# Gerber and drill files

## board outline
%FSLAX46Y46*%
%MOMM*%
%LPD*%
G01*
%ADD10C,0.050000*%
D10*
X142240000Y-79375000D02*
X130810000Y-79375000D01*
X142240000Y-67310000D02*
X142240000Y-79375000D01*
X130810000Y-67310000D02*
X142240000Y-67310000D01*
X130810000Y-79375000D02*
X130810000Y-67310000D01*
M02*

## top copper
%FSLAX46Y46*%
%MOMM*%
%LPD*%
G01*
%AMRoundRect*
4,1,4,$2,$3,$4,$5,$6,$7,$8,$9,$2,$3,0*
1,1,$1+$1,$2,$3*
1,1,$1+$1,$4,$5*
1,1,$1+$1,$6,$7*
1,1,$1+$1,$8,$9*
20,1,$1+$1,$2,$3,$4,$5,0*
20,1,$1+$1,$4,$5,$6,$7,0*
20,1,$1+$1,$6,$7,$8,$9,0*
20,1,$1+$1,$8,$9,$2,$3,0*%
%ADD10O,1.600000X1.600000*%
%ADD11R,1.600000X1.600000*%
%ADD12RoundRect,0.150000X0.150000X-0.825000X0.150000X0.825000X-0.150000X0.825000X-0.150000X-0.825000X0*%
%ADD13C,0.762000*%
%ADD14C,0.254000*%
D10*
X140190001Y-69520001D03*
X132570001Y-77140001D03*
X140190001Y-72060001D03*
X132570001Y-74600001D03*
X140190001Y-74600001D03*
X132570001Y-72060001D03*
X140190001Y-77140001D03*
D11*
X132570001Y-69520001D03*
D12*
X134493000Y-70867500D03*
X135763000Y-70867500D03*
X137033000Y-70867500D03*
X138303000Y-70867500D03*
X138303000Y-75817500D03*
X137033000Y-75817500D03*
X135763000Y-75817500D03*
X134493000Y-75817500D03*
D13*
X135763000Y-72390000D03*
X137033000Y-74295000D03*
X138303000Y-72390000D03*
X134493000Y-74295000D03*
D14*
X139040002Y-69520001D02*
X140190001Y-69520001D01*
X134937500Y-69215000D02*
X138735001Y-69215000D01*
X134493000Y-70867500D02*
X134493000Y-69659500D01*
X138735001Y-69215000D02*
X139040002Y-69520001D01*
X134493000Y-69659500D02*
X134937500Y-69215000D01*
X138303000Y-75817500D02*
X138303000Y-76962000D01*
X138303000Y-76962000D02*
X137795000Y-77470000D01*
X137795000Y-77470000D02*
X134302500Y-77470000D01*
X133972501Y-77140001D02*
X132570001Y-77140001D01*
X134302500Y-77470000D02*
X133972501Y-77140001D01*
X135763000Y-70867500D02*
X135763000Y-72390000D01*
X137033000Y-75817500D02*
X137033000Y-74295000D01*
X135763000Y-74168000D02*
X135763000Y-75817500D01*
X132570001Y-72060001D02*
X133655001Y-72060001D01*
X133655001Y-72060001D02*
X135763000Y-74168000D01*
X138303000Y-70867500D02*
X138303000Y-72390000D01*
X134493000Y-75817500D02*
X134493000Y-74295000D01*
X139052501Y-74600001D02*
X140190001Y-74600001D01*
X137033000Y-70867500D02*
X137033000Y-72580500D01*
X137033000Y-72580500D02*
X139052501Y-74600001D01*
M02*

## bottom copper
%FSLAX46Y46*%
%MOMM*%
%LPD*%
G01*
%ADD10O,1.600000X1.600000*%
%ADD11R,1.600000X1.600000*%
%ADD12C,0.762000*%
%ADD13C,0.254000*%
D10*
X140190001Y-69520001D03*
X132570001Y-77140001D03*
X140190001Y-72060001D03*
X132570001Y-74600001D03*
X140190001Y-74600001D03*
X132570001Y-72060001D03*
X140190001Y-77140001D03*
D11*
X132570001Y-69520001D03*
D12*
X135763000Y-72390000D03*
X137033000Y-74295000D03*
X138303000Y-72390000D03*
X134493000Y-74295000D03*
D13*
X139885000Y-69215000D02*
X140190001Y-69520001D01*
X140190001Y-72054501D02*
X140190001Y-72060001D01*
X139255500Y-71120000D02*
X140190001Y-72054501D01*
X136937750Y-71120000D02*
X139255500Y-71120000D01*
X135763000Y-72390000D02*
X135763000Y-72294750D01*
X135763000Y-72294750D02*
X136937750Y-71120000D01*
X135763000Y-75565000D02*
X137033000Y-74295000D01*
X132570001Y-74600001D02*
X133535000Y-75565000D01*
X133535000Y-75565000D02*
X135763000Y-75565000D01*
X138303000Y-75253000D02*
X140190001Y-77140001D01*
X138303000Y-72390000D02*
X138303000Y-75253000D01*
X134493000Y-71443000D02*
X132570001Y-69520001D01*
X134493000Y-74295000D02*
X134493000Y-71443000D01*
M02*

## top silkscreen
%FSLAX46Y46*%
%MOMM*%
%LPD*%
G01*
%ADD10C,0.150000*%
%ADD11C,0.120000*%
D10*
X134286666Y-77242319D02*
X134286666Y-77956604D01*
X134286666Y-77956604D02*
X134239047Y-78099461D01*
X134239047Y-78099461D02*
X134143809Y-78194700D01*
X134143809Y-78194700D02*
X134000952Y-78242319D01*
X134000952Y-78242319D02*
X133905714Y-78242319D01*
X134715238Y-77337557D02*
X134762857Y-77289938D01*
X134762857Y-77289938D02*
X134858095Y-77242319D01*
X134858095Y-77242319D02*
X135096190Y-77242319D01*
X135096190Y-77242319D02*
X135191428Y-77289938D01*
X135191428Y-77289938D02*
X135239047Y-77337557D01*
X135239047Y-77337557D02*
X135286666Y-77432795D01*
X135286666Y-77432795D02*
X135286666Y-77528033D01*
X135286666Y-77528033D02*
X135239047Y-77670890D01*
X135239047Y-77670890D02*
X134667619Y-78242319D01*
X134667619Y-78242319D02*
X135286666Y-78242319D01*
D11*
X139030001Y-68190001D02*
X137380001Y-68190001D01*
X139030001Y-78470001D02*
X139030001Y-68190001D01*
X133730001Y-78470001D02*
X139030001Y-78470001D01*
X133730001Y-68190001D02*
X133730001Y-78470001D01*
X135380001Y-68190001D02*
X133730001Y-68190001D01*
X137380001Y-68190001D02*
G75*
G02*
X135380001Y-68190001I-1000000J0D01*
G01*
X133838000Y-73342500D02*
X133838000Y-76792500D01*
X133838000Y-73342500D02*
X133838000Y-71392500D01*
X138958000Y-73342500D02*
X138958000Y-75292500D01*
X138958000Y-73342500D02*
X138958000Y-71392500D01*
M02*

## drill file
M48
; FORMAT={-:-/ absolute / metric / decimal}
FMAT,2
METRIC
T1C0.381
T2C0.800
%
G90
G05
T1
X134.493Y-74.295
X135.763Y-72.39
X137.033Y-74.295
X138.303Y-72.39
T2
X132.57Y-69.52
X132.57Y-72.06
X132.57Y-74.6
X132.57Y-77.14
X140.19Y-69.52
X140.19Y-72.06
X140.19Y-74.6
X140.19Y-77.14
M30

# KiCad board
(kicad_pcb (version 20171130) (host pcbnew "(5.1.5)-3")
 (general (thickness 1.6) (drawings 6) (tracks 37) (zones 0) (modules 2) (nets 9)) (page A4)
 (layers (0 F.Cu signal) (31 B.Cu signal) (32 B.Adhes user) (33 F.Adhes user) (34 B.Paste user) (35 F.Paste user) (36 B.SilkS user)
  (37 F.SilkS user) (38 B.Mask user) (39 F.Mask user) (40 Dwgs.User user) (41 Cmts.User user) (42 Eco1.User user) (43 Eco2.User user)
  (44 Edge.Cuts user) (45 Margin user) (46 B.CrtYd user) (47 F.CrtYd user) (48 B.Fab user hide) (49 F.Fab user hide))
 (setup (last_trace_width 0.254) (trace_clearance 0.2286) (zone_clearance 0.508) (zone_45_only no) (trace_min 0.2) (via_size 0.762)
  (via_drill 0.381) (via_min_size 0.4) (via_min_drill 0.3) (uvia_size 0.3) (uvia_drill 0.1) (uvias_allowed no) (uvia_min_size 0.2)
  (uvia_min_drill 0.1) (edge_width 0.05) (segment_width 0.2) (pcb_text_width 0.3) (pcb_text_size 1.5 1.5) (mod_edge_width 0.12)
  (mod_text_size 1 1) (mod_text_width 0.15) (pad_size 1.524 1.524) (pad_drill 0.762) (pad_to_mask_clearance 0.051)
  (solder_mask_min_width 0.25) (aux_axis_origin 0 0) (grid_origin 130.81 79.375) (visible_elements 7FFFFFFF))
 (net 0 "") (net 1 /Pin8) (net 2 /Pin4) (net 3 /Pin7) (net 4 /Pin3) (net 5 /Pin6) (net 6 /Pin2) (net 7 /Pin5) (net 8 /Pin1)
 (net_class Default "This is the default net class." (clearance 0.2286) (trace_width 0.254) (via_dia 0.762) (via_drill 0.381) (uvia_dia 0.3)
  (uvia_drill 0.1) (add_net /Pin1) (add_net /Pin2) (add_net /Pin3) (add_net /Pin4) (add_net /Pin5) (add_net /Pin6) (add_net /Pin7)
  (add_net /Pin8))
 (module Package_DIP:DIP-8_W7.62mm (layer F.Cu) (at 132.570001 69.520001)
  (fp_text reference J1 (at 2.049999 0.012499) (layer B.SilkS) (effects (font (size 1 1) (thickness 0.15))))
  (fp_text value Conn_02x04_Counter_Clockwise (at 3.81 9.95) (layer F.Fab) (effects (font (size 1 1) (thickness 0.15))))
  (fp_line (start 6.46 -1.33) (end 4.81 -1.33) (layer F.SilkS) (width 0.12))
  (fp_line (start 6.46 8.95) (end 6.46 -1.33) (layer F.SilkS) (width 0.12))
  (fp_line (start 1.16 8.95) (end 6.46 8.95) (layer F.SilkS) (width 0.12))
  (fp_line (start 1.16 -1.33) (end 1.16 8.95) (layer F.SilkS) (width 0.12))
  (fp_line (start 2.81 -1.33) (end 1.16 -1.33) (layer F.SilkS) (width 0.12))
  (fp_arc (start 3.81 -1.33) (end 2.81 -1.33) (angle -180) (layer F.SilkS) (width 0.12))
  (pad 8 thru_hole oval (at 7.62 0) (size 1.6 1.6) (drill 0.8) (layers *.Cu *.Mask) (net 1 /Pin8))
  (pad 4 thru_hole oval (at 0 7.62) (size 1.6 1.6) (drill 0.8) (layers *.Cu *.Mask) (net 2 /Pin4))
  (pad 7 thru_hole oval (at 7.62 2.54) (size 1.6 1.6) (drill 0.8) (layers *.Cu *.Mask) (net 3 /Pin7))
  (pad 3 thru_hole oval (at 0 5.08) (size 1.6 1.6) (drill 0.8) (layers *.Cu *.Mask) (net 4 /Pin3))
  (pad 6 thru_hole oval (at 7.62 5.08) (size 1.6 1.6) (drill 0.8) (layers *.Cu *.Mask) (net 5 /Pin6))
  (pad 2 thru_hole oval (at 0 2.54) (size 1.6 1.6) (drill 0.8) (layers *.Cu *.Mask) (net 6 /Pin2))
  (pad 5 thru_hole oval (at 7.62 7.62) (size 1.6 1.6) (drill 0.8) (layers *.Cu *.Mask) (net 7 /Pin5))
  (pad 1 thru_hole rect (at 0 0) (size 1.6 1.6) (drill 0.8) (layers *.Cu *.Mask) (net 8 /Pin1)))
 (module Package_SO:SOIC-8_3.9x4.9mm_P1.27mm (layer F.Cu) (at 136.398 73.3425 90)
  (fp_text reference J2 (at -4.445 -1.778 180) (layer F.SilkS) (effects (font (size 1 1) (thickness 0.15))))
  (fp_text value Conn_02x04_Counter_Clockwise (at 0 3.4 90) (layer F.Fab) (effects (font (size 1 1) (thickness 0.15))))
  (fp_line (start 0 -2.56) (end -3.45 -2.56) (layer F.SilkS) (width 0.12))
  (fp_line (start 0 -2.56) (end 1.95 -2.56) (layer F.SilkS) (width 0.12))
  (fp_line (start 0 2.56) (end -1.95 2.56) (layer F.SilkS) (width 0.12))
  (fp_line (start 0 2.56) (end 1.95 2.56) (layer F.SilkS) (width 0.12))
  (pad 8 smd roundrect (at 2.475 -1.905 90) (size 1.95 0.6) (layers F.Cu F.Paste F.Mask) (roundrect_rratio 0.25) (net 1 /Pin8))
  (pad 7 smd roundrect (at 2.475 -0.635 90) (size 1.95 0.6) (layers F.Cu F.Paste F.Mask) (roundrect_rratio 0.25) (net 3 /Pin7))
  (pad 6 smd roundrect (at 2.475 0.635 90) (size 1.95 0.6) (layers F.Cu F.Paste F.Mask) (roundrect_rratio 0.25) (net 5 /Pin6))
  (pad 5 smd roundrect (at 2.475 1.905 90) (size 1.95 0.6) (layers F.Cu F.Paste F.Mask) (roundrect_rratio 0.25) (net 7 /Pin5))
  (pad 4 smd roundrect (at -2.475 1.905 90) (size 1.95 0.6) (layers F.Cu F.Paste F.Mask) (roundrect_rratio 0.25) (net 2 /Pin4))
  (pad 3 smd roundrect (at -2.475 0.635 90) (size 1.95 0.6) (layers F.Cu F.Paste F.Mask) (roundrect_rratio 0.25) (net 4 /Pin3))
  (pad 2 smd roundrect (at -2.475 -0.635 90) (size 1.95 0.6) (layers F.Cu F.Paste F.Mask) (roundrect_rratio 0.25) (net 6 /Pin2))
  (pad 1 smd roundrect (at -2.475 -1.905 90) (size 1.95 0.6) (layers F.Cu F.Paste F.Mask) (roundrect_rratio 0.25) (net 8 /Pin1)))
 (gr_line (start 142.24 79.375) (end 130.81 79.375) (layer Edge.Cuts) (width 0.05))
 (gr_line (start 142.24 67.31) (end 142.24 79.375) (layer Edge.Cuts) (width 0.05))
 (gr_line (start 130.81 67.31) (end 142.24 67.31) (layer Edge.Cuts) (width 0.05))
 (gr_line (start 130.81 79.375) (end 130.81 67.31) (layer Edge.Cuts) (width 0.05))
 (segment (start 139.885 69.215) (end 140.190001 69.520001) (width 0.254) (layer B.Cu) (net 1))
 (segment (start 139.040002 69.520001) (end 140.190001 69.520001) (width 0.254) (layer F.Cu) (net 1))
 (segment (start 134.9375 69.215) (end 138.735001 69.215) (width 0.254) (layer F.Cu) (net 1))
 (segment (start 134.493 70.8675) (end 134.493 69.6595) (width 0.254) (layer F.Cu) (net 1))
 (segment (start 138.735001 69.215) (end 139.040002 69.520001) (width 0.254) (layer F.Cu) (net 1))
 (segment (start 134.493 69.6595) (end 134.9375 69.215) (width 0.254) (layer F.Cu) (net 1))
 (segment (start 138.303 75.8175) (end 138.303 76.962) (width 0.254) (layer F.Cu) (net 2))
 (segment (start 138.303 76.962) (end 137.795 77.47) (width 0.254) (layer F.Cu) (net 2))
 (segment (start 137.795 77.47) (end 134.3025 77.47) (width 0.254) (layer F.Cu) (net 2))
 (segment (start 133.972501 77.140001) (end 132.570001 77.140001) (width 0.254) (layer F.Cu) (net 2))
 (segment (start 134.3025 77.47) (end 133.972501 77.140001) (width 0.254) (layer F.Cu) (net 2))
 (via (at 135.763 72.39) (size 0.762) (drill 0.381) (layers F.Cu B.Cu) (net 3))
 (segment (start 135.763 70.8675) (end 135.763 72.39) (width 0.254) (layer F.Cu) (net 3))
 (segment (start 140.190001 72.054501) (end 140.190001 72.060001) (width 0.254) (layer B.Cu) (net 3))
 (segment (start 139.2555 71.12) (end 140.190001 72.054501) (width 0.254) (layer B.Cu) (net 3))
 (segment (start 136.93775 71.12) (end 139.2555 71.12) (width 0.254) (layer B.Cu) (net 3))
 (segment (start 135.763 72.39) (end 135.763 72.29475) (width 0.254) (layer B.Cu) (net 3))
 (segment (start 135.763 72.29475) (end 136.93775 71.12) (width 0.254) (layer B.Cu) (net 3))
 (segment (start 137.033 75.8175) (end 137.033 74.295) (width 0.254) (layer F.Cu) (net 4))
 (via (at 137.033 74.295) (size 0.762) (drill 0.381) (layers F.Cu B.Cu) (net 4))
 (segment (start 135.763 75.565) (end 137.033 74.295) (width 0.254) (layer B.Cu) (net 4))
 (segment (start 132.570001 74.600001) (end 133.535 75.565) (width 0.254) (layer B.Cu) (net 4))
 (segment (start 133.535 75.565) (end 135.763 75.565) (width 0.254) (layer B.Cu) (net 4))
 (segment (start 135.763 74.168) (end 135.763 75.8175) (width 0.254) (layer F.Cu) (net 6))
 (segment (start 132.570001 72.060001) (end 133.655001 72.060001) (width 0.254) (layer F.Cu) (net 6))
 (segment (start 133.655001 72.060001) (end 135.763 74.168) (width 0.254) (layer F.Cu) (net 6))
 (segment (start 138.303 75.253) (end 140.190001 77.140001) (width 0.254) (layer B.Cu) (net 7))
 (via (at 138.303 72.39) (size 0.762) (drill 0.381) (layers F.Cu B.Cu) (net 7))
 (segment (start 138.303 72.39) (end 138.303 75.253) (width 0.254) (layer B.Cu) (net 7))
 (segment (start 138.303 70.8675) (end 138.303 72.39) (width 0.254) (layer F.Cu) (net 7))
 (segment (start 134.493 71.443) (end 132.570001 69.520001) (width 0.254) (layer B.Cu) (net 8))
 (via (at 134.493 74.295) (size 0.762) (drill 0.381) (layers F.Cu B.Cu) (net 8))
 (segment (start 134.493 74.295) (end 134.493 71.443) (width 0.254) (layer B.Cu) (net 8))
 (segment (start 134.493 75.8175) (end 134.493 74.295) (width 0.254) (layer F.Cu) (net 8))
 (segment (start 139.052501 74.600001) (end 140.190001 74.600001) (width 0.254) (layer F.Cu) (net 5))
 (segment (start 137.033 70.8675) (end 137.033 72.5805) (width 0.254) (layer F.Cu) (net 5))
 (segment (start 137.033 72.5805) (end 139.052501 74.600001) (width 0.254) (layer F.Cu) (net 5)))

